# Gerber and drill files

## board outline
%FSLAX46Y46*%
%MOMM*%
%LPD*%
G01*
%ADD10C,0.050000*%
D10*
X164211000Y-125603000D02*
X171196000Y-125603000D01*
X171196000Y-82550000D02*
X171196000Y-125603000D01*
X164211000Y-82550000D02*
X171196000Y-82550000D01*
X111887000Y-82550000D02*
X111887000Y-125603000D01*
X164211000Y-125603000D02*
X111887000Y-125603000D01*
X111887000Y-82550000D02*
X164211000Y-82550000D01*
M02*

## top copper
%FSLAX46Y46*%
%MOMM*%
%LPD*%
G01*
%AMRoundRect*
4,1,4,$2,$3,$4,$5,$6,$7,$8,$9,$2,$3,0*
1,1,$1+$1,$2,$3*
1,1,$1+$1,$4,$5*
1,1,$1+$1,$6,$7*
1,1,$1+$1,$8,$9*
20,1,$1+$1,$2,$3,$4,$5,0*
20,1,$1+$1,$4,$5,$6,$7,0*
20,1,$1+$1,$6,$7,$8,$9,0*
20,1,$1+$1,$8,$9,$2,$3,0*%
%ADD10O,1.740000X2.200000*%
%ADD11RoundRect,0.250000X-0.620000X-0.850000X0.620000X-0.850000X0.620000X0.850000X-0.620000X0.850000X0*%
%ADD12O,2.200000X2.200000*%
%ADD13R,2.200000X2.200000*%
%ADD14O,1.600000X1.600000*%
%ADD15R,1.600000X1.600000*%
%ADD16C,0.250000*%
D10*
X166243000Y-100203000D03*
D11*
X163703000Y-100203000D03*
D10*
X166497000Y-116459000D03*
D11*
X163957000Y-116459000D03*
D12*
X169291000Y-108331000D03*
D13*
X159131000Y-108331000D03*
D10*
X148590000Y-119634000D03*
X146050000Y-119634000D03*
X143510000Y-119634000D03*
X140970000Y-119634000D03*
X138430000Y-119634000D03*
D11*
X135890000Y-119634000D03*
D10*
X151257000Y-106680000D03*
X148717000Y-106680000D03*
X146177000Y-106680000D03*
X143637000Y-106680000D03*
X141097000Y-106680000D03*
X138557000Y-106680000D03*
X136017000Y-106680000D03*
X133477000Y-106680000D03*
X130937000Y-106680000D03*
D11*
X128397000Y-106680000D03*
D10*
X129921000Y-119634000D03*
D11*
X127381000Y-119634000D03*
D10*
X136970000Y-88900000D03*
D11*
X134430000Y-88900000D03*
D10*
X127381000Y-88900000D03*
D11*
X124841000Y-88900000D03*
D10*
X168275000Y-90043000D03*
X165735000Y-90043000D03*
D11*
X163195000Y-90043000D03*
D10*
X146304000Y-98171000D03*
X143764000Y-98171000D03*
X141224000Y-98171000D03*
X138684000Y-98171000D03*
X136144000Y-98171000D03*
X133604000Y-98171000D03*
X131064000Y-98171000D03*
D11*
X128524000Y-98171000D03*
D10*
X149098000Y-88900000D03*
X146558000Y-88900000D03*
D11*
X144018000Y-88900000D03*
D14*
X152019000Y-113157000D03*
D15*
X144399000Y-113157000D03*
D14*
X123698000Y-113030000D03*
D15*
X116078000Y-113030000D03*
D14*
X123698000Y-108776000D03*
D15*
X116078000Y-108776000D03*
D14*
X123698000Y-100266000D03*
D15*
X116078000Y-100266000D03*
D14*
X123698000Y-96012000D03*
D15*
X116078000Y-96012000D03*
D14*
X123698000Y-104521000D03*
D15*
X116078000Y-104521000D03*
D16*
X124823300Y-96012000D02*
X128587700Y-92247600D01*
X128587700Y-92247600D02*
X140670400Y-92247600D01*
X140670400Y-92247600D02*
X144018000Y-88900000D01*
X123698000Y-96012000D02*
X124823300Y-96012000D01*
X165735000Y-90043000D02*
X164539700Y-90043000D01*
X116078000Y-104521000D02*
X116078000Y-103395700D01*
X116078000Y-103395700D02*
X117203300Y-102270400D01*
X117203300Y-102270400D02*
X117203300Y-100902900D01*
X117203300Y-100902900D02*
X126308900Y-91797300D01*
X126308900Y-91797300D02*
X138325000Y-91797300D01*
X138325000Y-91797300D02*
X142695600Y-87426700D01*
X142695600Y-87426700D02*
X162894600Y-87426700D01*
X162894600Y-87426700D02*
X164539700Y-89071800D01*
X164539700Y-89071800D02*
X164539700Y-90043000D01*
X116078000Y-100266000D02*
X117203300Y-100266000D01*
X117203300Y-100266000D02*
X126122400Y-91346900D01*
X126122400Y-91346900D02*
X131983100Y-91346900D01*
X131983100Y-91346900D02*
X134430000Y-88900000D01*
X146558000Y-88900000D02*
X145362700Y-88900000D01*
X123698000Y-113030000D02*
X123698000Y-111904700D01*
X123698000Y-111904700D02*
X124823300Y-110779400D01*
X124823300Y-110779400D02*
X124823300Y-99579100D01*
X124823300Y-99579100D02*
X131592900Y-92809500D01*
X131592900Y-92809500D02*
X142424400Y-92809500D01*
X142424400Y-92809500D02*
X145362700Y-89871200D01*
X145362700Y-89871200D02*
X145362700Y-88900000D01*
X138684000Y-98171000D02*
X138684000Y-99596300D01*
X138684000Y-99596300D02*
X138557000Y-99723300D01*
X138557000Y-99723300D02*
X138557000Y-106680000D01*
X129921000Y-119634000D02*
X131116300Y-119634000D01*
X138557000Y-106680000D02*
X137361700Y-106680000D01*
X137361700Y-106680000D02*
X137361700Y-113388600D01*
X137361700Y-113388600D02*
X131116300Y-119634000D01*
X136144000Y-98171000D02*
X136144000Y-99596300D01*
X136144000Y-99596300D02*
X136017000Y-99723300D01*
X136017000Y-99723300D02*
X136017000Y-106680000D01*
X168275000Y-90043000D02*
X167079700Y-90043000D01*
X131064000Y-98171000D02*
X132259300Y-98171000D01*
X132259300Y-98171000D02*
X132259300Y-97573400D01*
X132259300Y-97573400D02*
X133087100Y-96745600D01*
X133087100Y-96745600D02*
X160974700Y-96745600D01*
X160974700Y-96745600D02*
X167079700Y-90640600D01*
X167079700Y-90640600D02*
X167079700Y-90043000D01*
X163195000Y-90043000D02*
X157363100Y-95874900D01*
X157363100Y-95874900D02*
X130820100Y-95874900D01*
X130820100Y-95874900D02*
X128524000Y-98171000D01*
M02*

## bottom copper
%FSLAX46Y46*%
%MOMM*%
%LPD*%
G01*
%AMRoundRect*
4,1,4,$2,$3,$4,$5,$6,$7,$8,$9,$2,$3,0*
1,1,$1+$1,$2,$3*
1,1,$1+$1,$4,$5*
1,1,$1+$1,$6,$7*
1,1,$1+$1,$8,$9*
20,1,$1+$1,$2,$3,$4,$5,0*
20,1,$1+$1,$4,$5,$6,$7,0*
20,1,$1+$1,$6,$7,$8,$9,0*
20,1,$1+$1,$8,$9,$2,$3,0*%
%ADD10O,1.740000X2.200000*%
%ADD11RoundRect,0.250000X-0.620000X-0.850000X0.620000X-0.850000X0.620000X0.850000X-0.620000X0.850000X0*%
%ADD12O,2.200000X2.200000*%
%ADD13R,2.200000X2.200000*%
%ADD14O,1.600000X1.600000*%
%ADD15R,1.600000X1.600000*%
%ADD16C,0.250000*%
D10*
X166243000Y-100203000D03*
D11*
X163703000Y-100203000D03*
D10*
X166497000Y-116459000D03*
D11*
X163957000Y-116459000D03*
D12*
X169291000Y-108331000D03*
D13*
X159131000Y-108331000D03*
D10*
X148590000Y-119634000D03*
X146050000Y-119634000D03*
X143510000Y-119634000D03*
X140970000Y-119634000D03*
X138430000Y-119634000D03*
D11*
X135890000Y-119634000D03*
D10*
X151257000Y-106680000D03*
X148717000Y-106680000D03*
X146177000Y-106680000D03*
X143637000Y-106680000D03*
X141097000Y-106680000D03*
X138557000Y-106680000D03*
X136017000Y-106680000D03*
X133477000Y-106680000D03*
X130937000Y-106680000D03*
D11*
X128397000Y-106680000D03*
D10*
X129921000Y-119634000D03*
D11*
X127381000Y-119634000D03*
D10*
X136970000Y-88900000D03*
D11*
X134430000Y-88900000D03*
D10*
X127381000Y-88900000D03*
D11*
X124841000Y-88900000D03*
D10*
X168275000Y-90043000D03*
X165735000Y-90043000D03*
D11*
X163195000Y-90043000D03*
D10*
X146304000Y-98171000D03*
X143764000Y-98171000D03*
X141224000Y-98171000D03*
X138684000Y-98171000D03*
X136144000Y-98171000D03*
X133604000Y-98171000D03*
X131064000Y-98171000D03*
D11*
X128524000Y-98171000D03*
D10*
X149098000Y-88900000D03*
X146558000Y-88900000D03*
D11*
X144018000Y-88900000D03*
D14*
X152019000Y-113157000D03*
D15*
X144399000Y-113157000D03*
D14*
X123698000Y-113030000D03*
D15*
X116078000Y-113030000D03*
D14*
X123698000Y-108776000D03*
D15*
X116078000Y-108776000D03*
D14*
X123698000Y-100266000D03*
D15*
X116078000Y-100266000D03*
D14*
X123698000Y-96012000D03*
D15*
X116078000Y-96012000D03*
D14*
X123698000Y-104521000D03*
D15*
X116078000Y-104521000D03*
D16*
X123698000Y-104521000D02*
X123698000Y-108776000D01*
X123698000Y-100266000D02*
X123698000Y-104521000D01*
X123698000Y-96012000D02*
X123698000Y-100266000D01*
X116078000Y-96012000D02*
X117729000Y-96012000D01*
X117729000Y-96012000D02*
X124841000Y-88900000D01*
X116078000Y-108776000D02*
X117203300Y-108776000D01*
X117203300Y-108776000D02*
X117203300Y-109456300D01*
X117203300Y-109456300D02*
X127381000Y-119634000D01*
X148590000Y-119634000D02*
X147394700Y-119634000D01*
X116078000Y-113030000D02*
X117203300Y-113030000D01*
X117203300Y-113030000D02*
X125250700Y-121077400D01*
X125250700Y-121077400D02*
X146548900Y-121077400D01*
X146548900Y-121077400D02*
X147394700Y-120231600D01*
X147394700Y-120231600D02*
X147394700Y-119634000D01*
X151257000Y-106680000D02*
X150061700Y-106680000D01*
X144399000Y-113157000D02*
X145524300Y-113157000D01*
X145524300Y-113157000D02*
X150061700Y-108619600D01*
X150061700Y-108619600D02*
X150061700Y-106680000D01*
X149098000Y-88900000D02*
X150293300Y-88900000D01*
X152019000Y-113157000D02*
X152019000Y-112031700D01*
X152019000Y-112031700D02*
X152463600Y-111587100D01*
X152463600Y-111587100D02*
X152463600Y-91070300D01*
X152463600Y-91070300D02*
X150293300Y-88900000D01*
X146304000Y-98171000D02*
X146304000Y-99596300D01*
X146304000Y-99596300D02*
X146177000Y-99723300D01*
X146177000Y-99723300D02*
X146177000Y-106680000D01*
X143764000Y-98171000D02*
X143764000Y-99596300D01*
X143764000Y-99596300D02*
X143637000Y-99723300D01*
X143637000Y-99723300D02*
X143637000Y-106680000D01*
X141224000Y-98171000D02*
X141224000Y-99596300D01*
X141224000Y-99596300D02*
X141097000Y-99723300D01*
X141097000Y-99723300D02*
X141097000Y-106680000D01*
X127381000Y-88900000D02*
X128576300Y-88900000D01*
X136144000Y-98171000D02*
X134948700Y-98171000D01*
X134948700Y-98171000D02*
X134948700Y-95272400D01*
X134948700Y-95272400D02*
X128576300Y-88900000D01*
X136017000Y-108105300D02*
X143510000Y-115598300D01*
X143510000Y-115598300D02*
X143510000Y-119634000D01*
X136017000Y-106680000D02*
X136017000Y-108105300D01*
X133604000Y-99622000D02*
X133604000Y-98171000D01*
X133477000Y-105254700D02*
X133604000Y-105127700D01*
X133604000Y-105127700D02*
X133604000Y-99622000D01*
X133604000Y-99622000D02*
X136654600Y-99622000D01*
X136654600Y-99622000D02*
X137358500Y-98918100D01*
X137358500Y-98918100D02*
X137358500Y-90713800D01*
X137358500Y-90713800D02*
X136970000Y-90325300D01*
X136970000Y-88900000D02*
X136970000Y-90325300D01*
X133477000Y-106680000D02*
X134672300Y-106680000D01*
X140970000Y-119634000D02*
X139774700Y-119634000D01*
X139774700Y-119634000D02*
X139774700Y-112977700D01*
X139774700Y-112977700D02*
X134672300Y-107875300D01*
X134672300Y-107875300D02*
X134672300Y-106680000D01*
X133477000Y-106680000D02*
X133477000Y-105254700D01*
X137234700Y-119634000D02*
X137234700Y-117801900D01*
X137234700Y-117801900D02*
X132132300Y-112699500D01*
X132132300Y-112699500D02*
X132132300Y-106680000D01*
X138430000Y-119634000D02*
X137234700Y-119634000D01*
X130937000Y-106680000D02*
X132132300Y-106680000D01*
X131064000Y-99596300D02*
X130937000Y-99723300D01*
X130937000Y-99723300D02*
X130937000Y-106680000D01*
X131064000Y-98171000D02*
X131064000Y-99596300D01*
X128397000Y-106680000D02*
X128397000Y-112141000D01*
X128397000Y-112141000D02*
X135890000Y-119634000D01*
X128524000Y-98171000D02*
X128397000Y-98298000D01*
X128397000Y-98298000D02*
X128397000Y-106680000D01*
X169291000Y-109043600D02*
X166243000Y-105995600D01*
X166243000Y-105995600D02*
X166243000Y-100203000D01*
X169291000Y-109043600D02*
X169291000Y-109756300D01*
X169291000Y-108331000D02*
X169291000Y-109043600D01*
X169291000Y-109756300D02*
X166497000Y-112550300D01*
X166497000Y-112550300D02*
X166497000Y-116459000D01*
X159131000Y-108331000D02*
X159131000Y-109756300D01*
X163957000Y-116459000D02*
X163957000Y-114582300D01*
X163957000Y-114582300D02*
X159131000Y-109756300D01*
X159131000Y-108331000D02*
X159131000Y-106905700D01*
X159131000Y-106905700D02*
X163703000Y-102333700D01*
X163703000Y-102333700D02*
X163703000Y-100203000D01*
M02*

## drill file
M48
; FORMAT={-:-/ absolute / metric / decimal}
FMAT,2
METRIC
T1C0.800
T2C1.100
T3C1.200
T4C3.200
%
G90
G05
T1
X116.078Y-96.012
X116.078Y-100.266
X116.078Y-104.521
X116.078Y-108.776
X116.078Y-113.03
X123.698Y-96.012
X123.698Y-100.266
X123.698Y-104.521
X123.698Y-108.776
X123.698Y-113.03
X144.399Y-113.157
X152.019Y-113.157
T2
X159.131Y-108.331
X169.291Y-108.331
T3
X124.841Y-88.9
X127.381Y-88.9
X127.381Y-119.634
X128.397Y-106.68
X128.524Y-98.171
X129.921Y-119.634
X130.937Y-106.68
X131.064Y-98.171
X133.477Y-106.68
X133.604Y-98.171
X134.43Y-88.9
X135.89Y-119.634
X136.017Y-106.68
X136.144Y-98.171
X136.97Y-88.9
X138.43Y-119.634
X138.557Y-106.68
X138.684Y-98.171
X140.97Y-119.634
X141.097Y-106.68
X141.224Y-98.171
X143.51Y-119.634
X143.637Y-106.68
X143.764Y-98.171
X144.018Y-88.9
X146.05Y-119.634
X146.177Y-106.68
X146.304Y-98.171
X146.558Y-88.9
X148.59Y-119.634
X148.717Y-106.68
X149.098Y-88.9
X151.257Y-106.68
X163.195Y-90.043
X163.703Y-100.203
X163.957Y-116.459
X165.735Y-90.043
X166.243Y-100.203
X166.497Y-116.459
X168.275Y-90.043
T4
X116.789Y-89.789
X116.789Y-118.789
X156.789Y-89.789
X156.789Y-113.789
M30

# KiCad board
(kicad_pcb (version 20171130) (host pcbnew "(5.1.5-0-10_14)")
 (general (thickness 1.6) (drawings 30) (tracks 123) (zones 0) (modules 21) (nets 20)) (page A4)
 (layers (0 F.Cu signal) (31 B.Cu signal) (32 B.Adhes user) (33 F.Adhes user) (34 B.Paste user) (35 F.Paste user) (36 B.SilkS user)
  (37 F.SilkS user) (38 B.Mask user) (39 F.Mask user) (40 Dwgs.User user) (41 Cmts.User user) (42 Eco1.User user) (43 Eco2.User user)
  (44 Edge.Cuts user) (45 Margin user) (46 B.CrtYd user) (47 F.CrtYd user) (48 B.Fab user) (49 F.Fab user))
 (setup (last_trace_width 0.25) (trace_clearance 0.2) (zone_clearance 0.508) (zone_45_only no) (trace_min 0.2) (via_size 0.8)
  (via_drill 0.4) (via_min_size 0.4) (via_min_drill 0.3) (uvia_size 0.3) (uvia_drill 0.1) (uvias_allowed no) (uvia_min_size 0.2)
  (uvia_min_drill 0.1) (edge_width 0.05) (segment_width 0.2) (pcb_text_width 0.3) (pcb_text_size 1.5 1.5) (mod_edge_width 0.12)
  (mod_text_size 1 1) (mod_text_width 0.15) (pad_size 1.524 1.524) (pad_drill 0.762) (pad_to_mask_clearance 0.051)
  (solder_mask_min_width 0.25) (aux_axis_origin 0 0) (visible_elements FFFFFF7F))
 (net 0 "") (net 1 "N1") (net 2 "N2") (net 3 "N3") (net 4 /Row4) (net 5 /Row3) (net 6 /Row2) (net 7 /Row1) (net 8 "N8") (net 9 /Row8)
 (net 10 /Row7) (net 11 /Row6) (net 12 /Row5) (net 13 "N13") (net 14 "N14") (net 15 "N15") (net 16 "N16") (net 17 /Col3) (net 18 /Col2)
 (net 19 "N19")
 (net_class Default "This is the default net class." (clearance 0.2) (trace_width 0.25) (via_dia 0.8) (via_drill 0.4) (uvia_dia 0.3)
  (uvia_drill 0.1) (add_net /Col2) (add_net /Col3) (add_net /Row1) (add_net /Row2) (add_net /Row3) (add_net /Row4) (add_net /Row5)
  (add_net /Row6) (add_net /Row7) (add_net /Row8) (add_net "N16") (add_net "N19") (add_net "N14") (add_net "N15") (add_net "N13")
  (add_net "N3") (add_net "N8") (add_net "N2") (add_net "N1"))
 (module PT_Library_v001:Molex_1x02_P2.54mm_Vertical (layer F.Cu) (at 163.703 100.203)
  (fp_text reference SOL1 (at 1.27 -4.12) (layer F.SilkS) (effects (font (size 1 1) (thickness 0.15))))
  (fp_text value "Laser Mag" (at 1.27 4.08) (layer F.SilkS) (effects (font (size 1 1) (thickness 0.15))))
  (pad 2 thru_hole oval (at 2.54 0) (size 1.74 2.2) (drill 1.2) (layers *.Cu *.Mask) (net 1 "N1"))
  (pad 1 thru_hole roundrect (at 0 0) (size 1.74 2.2) (drill 1.2) (layers *.Cu *.Mask) (roundrect_rratio 0.143678) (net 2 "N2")))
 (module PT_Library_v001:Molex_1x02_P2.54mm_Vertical (layer F.Cu) (at 163.957 116.459)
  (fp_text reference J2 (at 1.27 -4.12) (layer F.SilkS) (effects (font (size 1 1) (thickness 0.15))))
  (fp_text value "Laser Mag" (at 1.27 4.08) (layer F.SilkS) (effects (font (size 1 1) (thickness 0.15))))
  (pad 2 thru_hole oval (at 2.54 0) (size 1.74 2.2) (drill 1.2) (layers *.Cu *.Mask) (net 1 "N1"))
  (pad 1 thru_hole roundrect (at 0 0) (size 1.74 2.2) (drill 1.2) (layers *.Cu *.Mask) (roundrect_rratio 0.143678) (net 2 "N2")))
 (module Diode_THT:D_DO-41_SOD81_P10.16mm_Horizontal (layer F.Cu) (at 159.131 108.331)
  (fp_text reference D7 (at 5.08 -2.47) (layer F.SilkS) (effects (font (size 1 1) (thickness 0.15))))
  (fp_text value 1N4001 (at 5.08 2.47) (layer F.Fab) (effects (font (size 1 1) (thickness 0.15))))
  (pad 2 thru_hole oval (at 10.16 0) (size 2.2 2.2) (drill 1.1) (layers *.Cu *.Mask) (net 1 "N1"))
  (pad 1 thru_hole rect (at 0 0) (size 2.2 2.2) (drill 1.1) (layers *.Cu *.Mask) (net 2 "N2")))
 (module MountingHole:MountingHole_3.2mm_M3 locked (layer F.Cu) (at 116.789 89.789)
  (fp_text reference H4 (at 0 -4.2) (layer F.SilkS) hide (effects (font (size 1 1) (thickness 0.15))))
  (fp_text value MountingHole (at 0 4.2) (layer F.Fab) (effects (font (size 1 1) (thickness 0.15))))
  (pad 1 np_thru_hole circle (at 0 0) (size 3.2 3.2) (drill 3.2) (layers *.Cu *.Mask)))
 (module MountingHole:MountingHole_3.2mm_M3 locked (layer F.Cu) (at 156.789 89.789)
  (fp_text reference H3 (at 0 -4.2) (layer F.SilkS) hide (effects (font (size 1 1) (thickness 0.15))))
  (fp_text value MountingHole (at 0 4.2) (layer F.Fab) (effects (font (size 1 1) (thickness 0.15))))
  (pad 1 np_thru_hole circle (at 0 0) (size 3.2 3.2) (drill 3.2) (layers *.Cu *.Mask)))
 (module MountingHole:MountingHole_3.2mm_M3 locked (layer F.Cu) (at 156.789 113.789)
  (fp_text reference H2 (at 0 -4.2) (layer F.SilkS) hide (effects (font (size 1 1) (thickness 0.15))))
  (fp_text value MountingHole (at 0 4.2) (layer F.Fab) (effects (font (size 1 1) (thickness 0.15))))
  (pad 1 np_thru_hole circle (at 0 0) (size 3.2 3.2) (drill 3.2) (layers *.Cu *.Mask)))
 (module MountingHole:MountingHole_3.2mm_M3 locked (layer F.Cu) (at 116.789 118.789)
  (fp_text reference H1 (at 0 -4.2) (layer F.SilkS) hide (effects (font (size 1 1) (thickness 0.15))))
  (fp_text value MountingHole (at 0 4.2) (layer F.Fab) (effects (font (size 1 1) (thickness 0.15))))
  (pad 1 np_thru_hole circle (at 0 0) (size 3.2 3.2) (drill 3.2) (layers *.Cu *.Mask)))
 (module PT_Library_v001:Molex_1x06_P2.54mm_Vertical (layer F.Cu) (at 135.89 119.634)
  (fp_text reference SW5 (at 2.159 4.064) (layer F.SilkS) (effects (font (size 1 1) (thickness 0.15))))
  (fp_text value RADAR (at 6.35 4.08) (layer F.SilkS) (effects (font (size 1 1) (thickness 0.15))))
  (pad 6 thru_hole oval (at 12.7 0) (size 1.74 2.2) (drill 1.2) (layers *.Cu *.Mask) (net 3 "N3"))
  (pad 5 thru_hole oval (at 10.16 0) (size 1.74 2.2) (drill 1.2) (layers *.Cu *.Mask))
  (pad 4 thru_hole oval (at 7.62 0) (size 1.74 2.2) (drill 1.2) (layers *.Cu *.Mask) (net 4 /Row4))
  (pad 3 thru_hole oval (at 5.08 0) (size 1.74 2.2) (drill 1.2) (layers *.Cu *.Mask) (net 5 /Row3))
  (pad 2 thru_hole oval (at 2.54 0) (size 1.74 2.2) (drill 1.2) (layers *.Cu *.Mask) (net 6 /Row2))
  (pad 1 thru_hole roundrect (at 0 0) (size 1.74 2.2) (drill 1.2) (layers *.Cu *.Mask) (roundrect_rratio 0.143678) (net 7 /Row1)))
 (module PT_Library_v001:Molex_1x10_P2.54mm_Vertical (layer F.Cu) (at 128.397 106.68)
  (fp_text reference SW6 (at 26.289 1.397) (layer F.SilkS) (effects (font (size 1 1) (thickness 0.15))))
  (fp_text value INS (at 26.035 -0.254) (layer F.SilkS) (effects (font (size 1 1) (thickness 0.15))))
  (pad 10 thru_hole oval (at 22.86 0) (size 1.74 2.2) (drill 1.2) (layers *.Cu *.Mask) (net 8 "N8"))
  (pad 9 thru_hole oval (at 20.32 0) (size 1.74 2.2) (drill 1.2) (layers *.Cu *.Mask))
  (pad 8 thru_hole oval (at 17.78 0) (size 1.74 2.2) (drill 1.2) (layers *.Cu *.Mask) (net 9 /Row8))
  (pad 7 thru_hole oval (at 15.24 0) (size 1.74 2.2) (drill 1.2) (layers *.Cu *.Mask) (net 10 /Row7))
  (pad 6 thru_hole oval (at 12.7 0) (size 1.74 2.2) (drill 1.2) (layers *.Cu *.Mask) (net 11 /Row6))
  (pad 5 thru_hole oval (at 10.16 0) (size 1.74 2.2) (drill 1.2) (layers *.Cu *.Mask) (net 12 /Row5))
  (pad 4 thru_hole oval (at 7.62 0) (size 1.74 2.2) (drill 1.2) (layers *.Cu *.Mask) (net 4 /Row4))
  (pad 3 thru_hole oval (at 5.08 0) (size 1.74 2.2) (drill 1.2) (layers *.Cu *.Mask) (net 5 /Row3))
  (pad 2 thru_hole oval (at 2.54 0) (size 1.74 2.2) (drill 1.2) (layers *.Cu *.Mask) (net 6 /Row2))
  (pad 1 thru_hole roundrect (at 0 0) (size 1.74 2.2) (drill 1.2) (layers *.Cu *.Mask) (roundrect_rratio 0.143678) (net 7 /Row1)))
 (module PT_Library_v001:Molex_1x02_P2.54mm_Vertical (layer F.Cu) (at 127.381 119.634)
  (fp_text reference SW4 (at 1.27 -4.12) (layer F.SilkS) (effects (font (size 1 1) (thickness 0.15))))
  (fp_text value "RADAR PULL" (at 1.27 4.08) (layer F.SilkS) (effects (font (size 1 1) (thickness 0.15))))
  (pad 2 thru_hole oval (at 2.54 0) (size 1.74 2.2) (drill 1.2) (layers *.Cu *.Mask) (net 12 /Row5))
  (pad 1 thru_hole roundrect (at 0 0) (size 1.74 2.2) (drill 1.2) (layers *.Cu *.Mask) (roundrect_rratio 0.143678) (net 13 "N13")))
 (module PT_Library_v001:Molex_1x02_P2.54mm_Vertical (layer F.Cu) (at 134.43 88.9)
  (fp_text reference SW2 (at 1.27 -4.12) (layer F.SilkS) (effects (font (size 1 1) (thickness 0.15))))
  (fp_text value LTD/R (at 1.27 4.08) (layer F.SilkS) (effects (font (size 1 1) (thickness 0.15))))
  (pad 2 thru_hole oval (at 2.54 0) (size 1.74 2.2) (drill 1.2) (layers *.Cu *.Mask) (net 5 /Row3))
  (pad 1 thru_hole roundrect (at 0 0) (size 1.74 2.2) (drill 1.2) (layers *.Cu *.Mask) (roundrect_rratio 0.143678) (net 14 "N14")))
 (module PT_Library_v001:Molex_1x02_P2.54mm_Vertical (layer F.Cu) (at 124.841 88.9)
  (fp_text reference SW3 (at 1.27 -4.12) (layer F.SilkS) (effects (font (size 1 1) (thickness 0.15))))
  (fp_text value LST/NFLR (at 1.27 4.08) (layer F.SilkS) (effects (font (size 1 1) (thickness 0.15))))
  (pad 2 thru_hole oval (at 2.54 0) (size 1.74 2.2) (drill 1.2) (layers *.Cu *.Mask) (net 4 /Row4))
  (pad 1 thru_hole roundrect (at 0 0) (size 1.74 2.2) (drill 1.2) (layers *.Cu *.Mask) (roundrect_rratio 0.143678) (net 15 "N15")))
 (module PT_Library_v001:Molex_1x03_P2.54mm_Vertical (layer F.Cu) (at 163.195 90.043)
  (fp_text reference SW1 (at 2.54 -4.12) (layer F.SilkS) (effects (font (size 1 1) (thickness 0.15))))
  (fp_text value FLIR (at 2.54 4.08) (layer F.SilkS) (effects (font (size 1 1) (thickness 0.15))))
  (pad 3 thru_hole oval (at 5.08 0) (size 1.74 2.2) (drill 1.2) (layers *.Cu *.Mask) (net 6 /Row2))
  (pad 2 thru_hole oval (at 2.54 0) (size 1.74 2.2) (drill 1.2) (layers *.Cu *.Mask) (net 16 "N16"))
  (pad 1 thru_hole roundrect (at 0 0) (size 1.74 2.2) (drill 1.2) (layers *.Cu *.Mask) (roundrect_rratio 0.143678) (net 7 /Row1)))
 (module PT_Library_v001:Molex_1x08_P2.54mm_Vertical (layer F.Cu) (at 128.524 98.171)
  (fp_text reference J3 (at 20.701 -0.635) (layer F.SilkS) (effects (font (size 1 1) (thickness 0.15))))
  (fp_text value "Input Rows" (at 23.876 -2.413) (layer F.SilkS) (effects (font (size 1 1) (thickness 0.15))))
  (pad 8 thru_hole oval (at 17.78 0) (size 1.74 2.2) (drill 1.2) (layers *.Cu *.Mask) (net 9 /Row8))
  (pad 7 thru_hole oval (at 15.24 0) (size 1.74 2.2) (drill 1.2) (layers *.Cu *.Mask) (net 10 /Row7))
  (pad 6 thru_hole oval (at 12.7 0) (size 1.74 2.2) (drill 1.2) (layers *.Cu *.Mask) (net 11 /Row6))
  (pad 5 thru_hole oval (at 10.16 0) (size 1.74 2.2) (drill 1.2) (layers *.Cu *.Mask) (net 12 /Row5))
  (pad 4 thru_hole oval (at 7.62 0) (size 1.74 2.2) (drill 1.2) (layers *.Cu *.Mask) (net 4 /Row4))
  (pad 3 thru_hole oval (at 5.08 0) (size 1.74 2.2) (drill 1.2) (layers *.Cu *.Mask) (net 5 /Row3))
  (pad 2 thru_hole oval (at 2.54 0) (size 1.74 2.2) (drill 1.2) (layers *.Cu *.Mask) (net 6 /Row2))
  (pad 1 thru_hole roundrect (at 0 0) (size 1.74 2.2) (drill 1.2) (layers *.Cu *.Mask) (roundrect_rratio 0.143678) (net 7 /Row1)))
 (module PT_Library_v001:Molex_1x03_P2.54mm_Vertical (layer F.Cu) (at 144.018 88.9)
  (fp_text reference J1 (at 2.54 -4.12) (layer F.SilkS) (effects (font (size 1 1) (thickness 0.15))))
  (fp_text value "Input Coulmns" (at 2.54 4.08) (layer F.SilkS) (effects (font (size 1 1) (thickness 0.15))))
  (pad 3 thru_hole oval (at 5.08 0) (size 1.74 2.2) (drill 1.2) (layers *.Cu *.Mask) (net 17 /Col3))
  (pad 2 thru_hole oval (at 2.54 0) (size 1.74 2.2) (drill 1.2) (layers *.Cu *.Mask) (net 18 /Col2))
  (pad 1 thru_hole roundrect (at 0 0) (size 1.74 2.2) (drill 1.2) (layers *.Cu *.Mask) (roundrect_rratio 0.143678) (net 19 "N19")))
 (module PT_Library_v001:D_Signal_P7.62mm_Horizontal (layer F.Cu) (at 144.399 113.157)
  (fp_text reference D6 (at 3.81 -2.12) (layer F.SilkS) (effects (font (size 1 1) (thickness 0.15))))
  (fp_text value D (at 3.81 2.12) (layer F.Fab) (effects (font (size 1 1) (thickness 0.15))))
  (pad 2 thru_hole oval (at 7.62 0) (size 1.6 1.6) (drill 0.8) (layers *.Cu *.Mask) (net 17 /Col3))
  (pad 1 thru_hole rect (at 0 0) (size 1.6 1.6) (drill 0.8) (layers *.Cu *.Mask) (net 8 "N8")))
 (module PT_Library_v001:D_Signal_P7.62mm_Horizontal (layer F.Cu) (at 116.078 113.03)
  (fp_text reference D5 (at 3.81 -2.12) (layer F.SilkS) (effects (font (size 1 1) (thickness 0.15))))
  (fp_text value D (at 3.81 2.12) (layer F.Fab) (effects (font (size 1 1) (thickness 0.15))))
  (pad 2 thru_hole oval (at 7.62 0) (size 1.6 1.6) (drill 0.8) (layers *.Cu *.Mask) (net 18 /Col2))
  (pad 1 thru_hole rect (at 0 0) (size 1.6 1.6) (drill 0.8) (layers *.Cu *.Mask) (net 3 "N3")))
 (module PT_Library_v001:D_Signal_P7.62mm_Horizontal (layer F.Cu) (at 116.078 108.776)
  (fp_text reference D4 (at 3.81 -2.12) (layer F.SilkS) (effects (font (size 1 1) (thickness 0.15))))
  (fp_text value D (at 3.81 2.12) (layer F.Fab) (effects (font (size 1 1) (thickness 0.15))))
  (pad 2 thru_hole oval (at 7.62 0) (size 1.6 1.6) (drill 0.8) (layers *.Cu *.Mask) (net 19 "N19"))
  (pad 1 thru_hole rect (at 0 0) (size 1.6 1.6) (drill 0.8) (layers *.Cu *.Mask) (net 13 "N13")))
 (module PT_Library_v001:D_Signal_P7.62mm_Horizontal (layer F.Cu) (at 116.078 100.266)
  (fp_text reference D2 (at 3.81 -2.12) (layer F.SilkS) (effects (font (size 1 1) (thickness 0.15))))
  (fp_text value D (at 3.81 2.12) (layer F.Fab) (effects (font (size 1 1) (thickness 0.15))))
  (pad 2 thru_hole oval (at 7.62 0) (size 1.6 1.6) (drill 0.8) (layers *.Cu *.Mask) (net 19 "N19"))
  (pad 1 thru_hole rect (at 0 0) (size 1.6 1.6) (drill 0.8) (layers *.Cu *.Mask) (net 14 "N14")))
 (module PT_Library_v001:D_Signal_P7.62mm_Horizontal (layer F.Cu) (at 116.078 96.012)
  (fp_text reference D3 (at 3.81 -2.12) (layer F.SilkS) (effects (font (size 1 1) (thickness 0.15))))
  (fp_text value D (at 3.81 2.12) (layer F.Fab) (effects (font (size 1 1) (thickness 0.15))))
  (pad 2 thru_hole oval (at 7.62 0) (size 1.6 1.6) (drill 0.8) (layers *.Cu *.Mask) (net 19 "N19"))
  (pad 1 thru_hole rect (at 0 0) (size 1.6 1.6) (drill 0.8) (layers *.Cu *.Mask) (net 15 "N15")))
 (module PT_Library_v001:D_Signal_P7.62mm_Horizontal (layer F.Cu) (at 116.078 104.521)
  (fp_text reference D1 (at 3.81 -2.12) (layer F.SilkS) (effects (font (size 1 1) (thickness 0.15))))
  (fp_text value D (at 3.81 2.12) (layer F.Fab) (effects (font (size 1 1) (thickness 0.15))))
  (pad 2 thru_hole oval (at 7.62 0) (size 1.6 1.6) (drill 0.8) (layers *.Cu *.Mask) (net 19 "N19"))
  (pad 1 thru_hole rect (at 0 0) (size 1.6 1.6) (drill 0.8) (layers *.Cu *.Mask) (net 16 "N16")))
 (gr_line (start 164.211 125.603) (end 171.196 125.603) (layer Edge.Cuts) (width 0.05))
 (gr_line (start 171.196 82.55) (end 171.196 125.603) (layer Edge.Cuts) (width 0.05))
 (gr_line (start 164.211 82.55) (end 171.196 82.55) (layer Edge.Cuts) (width 0.05))
 (gr_line (start 111.887 82.55) (end 111.887 125.603) (layer Edge.Cuts) (width 0.05))
 (gr_line (start 164.211 125.603) (end 111.887 125.603) (layer Edge.Cuts) (width 0.05))
 (gr_line (start 111.887 82.55) (end 164.211 82.55) (layer Edge.Cuts) (width 0.05))
 (segment (start 124.8233 96.012) (end 128.5877 92.2476) (width 0.25) (layer F.Cu) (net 19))
 (segment (start 128.5877 92.2476) (end 140.6704 92.2476) (width 0.25) (layer F.Cu) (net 19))
 (segment (start 140.6704 92.2476) (end 144.018 88.9) (width 0.25) (layer F.Cu) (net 19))
 (segment (start 123.698 96.012) (end 124.8233 96.012) (width 0.25) (layer F.Cu) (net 19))
 (segment (start 123.698 104.521) (end 123.698 108.776) (width 0.25) (layer B.Cu) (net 19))
 (segment (start 123.698 100.266) (end 123.698 104.521) (width 0.25) (layer B.Cu) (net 19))
 (segment (start 123.698 96.012) (end 123.698 100.266) (width 0.25) (layer B.Cu) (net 19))
 (segment (start 165.735 90.043) (end 164.5397 90.043) (width 0.25) (layer F.Cu) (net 16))
 (segment (start 116.078 104.521) (end 116.078 103.3957) (width 0.25) (layer F.Cu) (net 16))
 (segment (start 116.078 103.3957) (end 117.2033 102.2704) (width 0.25) (layer F.Cu) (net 16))
 (segment (start 117.2033 102.2704) (end 117.2033 100.9029) (width 0.25) (layer F.Cu) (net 16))
 (segment (start 117.2033 100.9029) (end 126.3089 91.7973) (width 0.25) (layer F.Cu) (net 16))
 (segment (start 126.3089 91.7973) (end 138.325 91.7973) (width 0.25) (layer F.Cu) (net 16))
 (segment (start 138.325 91.7973) (end 142.6956 87.4267) (width 0.25) (layer F.Cu) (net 16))
 (segment (start 142.6956 87.4267) (end 162.8946 87.4267) (width 0.25) (layer F.Cu) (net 16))
 (segment (start 162.8946 87.4267) (end 164.5397 89.0718) (width 0.25) (layer F.Cu) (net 16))
 (segment (start 164.5397 89.0718) (end 164.5397 90.043) (width 0.25) (layer F.Cu) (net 16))
 (segment (start 116.078 100.266) (end 117.2033 100.266) (width 0.25) (layer F.Cu) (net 14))
 (segment (start 117.2033 100.266) (end 126.1224 91.3469) (width 0.25) (layer F.Cu) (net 14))
 (segment (start 126.1224 91.3469) (end 131.9831 91.3469) (width 0.25) (layer F.Cu) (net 14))
 (segment (start 131.9831 91.3469) (end 134.43 88.9) (width 0.25) (layer F.Cu) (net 14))
 (segment (start 116.078 96.012) (end 117.729 96.012) (width 0.25) (layer B.Cu) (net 15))
 (segment (start 117.729 96.012) (end 124.841 88.9) (width 0.25) (layer B.Cu) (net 15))
 (segment (start 116.078 108.776) (end 117.2033 108.776) (width 0.25) (layer B.Cu) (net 13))
 (segment (start 117.2033 108.776) (end 117.2033 109.4563) (width 0.25) (layer B.Cu) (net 13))
 (segment (start 117.2033 109.4563) (end 127.381 119.634) (width 0.25) (layer B.Cu) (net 13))
 (segment (start 148.59 119.634) (end 147.3947 119.634) (width 0.25) (layer B.Cu) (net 3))
 (segment (start 116.078 113.03) (end 117.2033 113.03) (width 0.25) (layer B.Cu) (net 3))
 (segment (start 117.2033 113.03) (end 125.2507 121.0774) (width 0.25) (layer B.Cu) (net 3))
 (segment (start 125.2507 121.0774) (end 146.5489 121.0774) (width 0.25) (layer B.Cu) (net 3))
 (segment (start 146.5489 121.0774) (end 147.3947 120.2316) (width 0.25) (layer B.Cu) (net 3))
 (segment (start 147.3947 120.2316) (end 147.3947 119.634) (width 0.25) (layer B.Cu) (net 3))
 (segment (start 146.558 88.9) (end 145.3627 88.9) (width 0.25) (layer F.Cu) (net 18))
 (segment (start 123.698 113.03) (end 123.698 111.9047) (width 0.25) (layer F.Cu) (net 18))
 (segment (start 123.698 111.9047) (end 124.8233 110.7794) (width 0.25) (layer F.Cu) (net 18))
 (segment (start 124.8233 110.7794) (end 124.8233 99.5791) (width 0.25) (layer F.Cu) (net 18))
 (segment (start 124.8233 99.5791) (end 131.5929 92.8095) (width 0.25) (layer F.Cu) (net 18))
 (segment (start 131.5929 92.8095) (end 142.4244 92.8095) (width 0.25) (layer F.Cu) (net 18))
 (segment (start 142.4244 92.8095) (end 145.3627 89.8712) (width 0.25) (layer F.Cu) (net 18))
 (segment (start 145.3627 89.8712) (end 145.3627 88.9) (width 0.25) (layer F.Cu) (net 18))
 (segment (start 151.257 106.68) (end 150.0617 106.68) (width 0.25) (layer B.Cu) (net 8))
 (segment (start 144.399 113.157) (end 145.5243 113.157) (width 0.25) (layer B.Cu) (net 8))
 (segment (start 145.5243 113.157) (end 150.0617 108.6196) (width 0.25) (layer B.Cu) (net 8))
 (segment (start 150.0617 108.6196) (end 150.0617 106.68) (width 0.25) (layer B.Cu) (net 8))
 (segment (start 149.098 88.9) (end 150.2933 88.9) (width 0.25) (layer B.Cu) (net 17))
 (segment (start 152.019 113.157) (end 152.019 112.0317) (width 0.25) (layer B.Cu) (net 17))
 (segment (start 152.019 112.0317) (end 152.4636 111.5871) (width 0.25) (layer B.Cu) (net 17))
 (segment (start 152.4636 111.5871) (end 152.4636 91.0703) (width 0.25) (layer B.Cu) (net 17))
 (segment (start 152.4636 91.0703) (end 150.2933 88.9) (width 0.25) (layer B.Cu) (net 17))
 (segment (start 146.304 98.171) (end 146.304 99.5963) (width 0.25) (layer B.Cu) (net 9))
 (segment (start 146.304 99.5963) (end 146.177 99.7233) (width 0.25) (layer B.Cu) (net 9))
 (segment (start 146.177 99.7233) (end 146.177 106.68) (width 0.25) (layer B.Cu) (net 9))
 (segment (start 143.764 98.171) (end 143.764 99.5963) (width 0.25) (layer B.Cu) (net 10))
 (segment (start 143.764 99.5963) (end 143.637 99.7233) (width 0.25) (layer B.Cu) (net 10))
 (segment (start 143.637 99.7233) (end 143.637 106.68) (width 0.25) (layer B.Cu) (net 10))
 (segment (start 141.224 98.171) (end 141.224 99.5963) (width 0.25) (layer B.Cu) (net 11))
 (segment (start 141.224 99.5963) (end 141.097 99.7233) (width 0.25) (layer B.Cu) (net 11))
 (segment (start 141.097 99.7233) (end 141.097 106.68) (width 0.25) (layer B.Cu) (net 11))
 (segment (start 138.684 98.171) (end 138.684 99.5963) (width 0.25) (layer F.Cu) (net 12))
 (segment (start 138.684 99.5963) (end 138.557 99.7233) (width 0.25) (layer F.Cu) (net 12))
 (segment (start 138.557 99.7233) (end 138.557 106.68) (width 0.25) (layer F.Cu) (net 12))
 (segment (start 129.921 119.634) (end 131.1163 119.634) (width 0.25) (layer F.Cu) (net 12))
 (segment (start 138.557 106.68) (end 137.3617 106.68) (width 0.25) (layer F.Cu) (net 12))
 (segment (start 137.3617 106.68) (end 137.3617 113.3886) (width 0.25) (layer F.Cu) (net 12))
 (segment (start 137.3617 113.3886) (end 131.1163 119.634) (width 0.25) (layer F.Cu) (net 12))
 (segment (start 127.381 88.9) (end 128.5763 88.9) (width 0.25) (layer B.Cu) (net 4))
 (segment (start 136.144 98.171) (end 134.9487 98.171) (width 0.25) (layer B.Cu) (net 4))
 (segment (start 134.9487 98.171) (end 134.9487 95.2724) (width 0.25) (layer B.Cu) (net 4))
 (segment (start 134.9487 95.2724) (end 128.5763 88.9) (width 0.25) (layer B.Cu) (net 4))
 (segment (start 136.144 98.171) (end 136.144 99.5963) (width 0.25) (layer F.Cu) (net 4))
 (segment (start 136.144 99.5963) (end 136.017 99.7233) (width 0.25) (layer F.Cu) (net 4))
 (segment (start 136.017 99.7233) (end 136.017 106.68) (width 0.25) (layer F.Cu) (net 4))
 (segment (start 136.017 108.1053) (end 143.51 115.5983) (width 0.25) (layer B.Cu) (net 4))
 (segment (start 143.51 115.5983) (end 143.51 119.634) (width 0.25) (layer B.Cu) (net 4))
 (segment (start 136.017 106.68) (end 136.017 108.1053) (width 0.25) (layer B.Cu) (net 4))
 (segment (start 133.604 99.622) (end 133.604 98.171) (width 0.25) (layer B.Cu) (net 5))
 (segment (start 133.477 105.2547) (end 133.604 105.1277) (width 0.25) (layer B.Cu) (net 5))
 (segment (start 133.604 105.1277) (end 133.604 99.622) (width 0.25) (layer B.Cu) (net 5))
 (segment (start 133.604 99.622) (end 136.6546 99.622) (width 0.25) (layer B.Cu) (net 5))
 (segment (start 136.6546 99.622) (end 137.3585 98.9181) (width 0.25) (layer B.Cu) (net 5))
 (segment (start 137.3585 98.9181) (end 137.3585 90.7138) (width 0.25) (layer B.Cu) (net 5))
 (segment (start 137.3585 90.7138) (end 136.97 90.3253) (width 0.25) (layer B.Cu) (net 5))
 (segment (start 136.97 88.9) (end 136.97 90.3253) (width 0.25) (layer B.Cu) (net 5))
 (segment (start 133.477 106.68) (end 134.6723 106.68) (width 0.25) (layer B.Cu) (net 5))
 (segment (start 140.97 119.634) (end 139.7747 119.634) (width 0.25) (layer B.Cu) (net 5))
 (segment (start 139.7747 119.634) (end 139.7747 112.9777) (width 0.25) (layer B.Cu) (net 5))
 (segment (start 139.7747 112.9777) (end 134.6723 107.8753) (width 0.25) (layer B.Cu) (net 5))
 (segment (start 134.6723 107.8753) (end 134.6723 106.68) (width 0.25) (layer B.Cu) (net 5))
 (segment (start 133.477 106.68) (end 133.477 105.2547) (width 0.25) (layer B.Cu) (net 5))
 (segment (start 137.2347 119.634) (end 137.2347 117.8019) (width 0.25) (layer B.Cu) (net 6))
 (segment (start 137.2347 117.8019) (end 132.1323 112.6995) (width 0.25) (layer B.Cu) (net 6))
 (segment (start 132.1323 112.6995) (end 132.1323 106.68) (width 0.25) (layer B.Cu) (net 6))
 (segment (start 168.275 90.043) (end 167.0797 90.043) (width 0.25) (layer F.Cu) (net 6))
 (segment (start 131.064 98.171) (end 132.2593 98.171) (width 0.25) (layer F.Cu) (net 6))
 (segment (start 132.2593 98.171) (end 132.2593 97.5734) (width 0.25) (layer F.Cu) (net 6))
 (segment (start 132.2593 97.5734) (end 133.0871 96.7456) (width 0.25) (layer F.Cu) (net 6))
 (segment (start 133.0871 96.7456) (end 160.9747 96.7456) (width 0.25) (layer F.Cu) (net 6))
 (segment (start 160.9747 96.7456) (end 167.0797 90.6406) (width 0.25) (layer F.Cu) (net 6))
 (segment (start 167.0797 90.6406) (end 167.0797 90.043) (width 0.25) (layer F.Cu) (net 6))
 (segment (start 138.43 119.634) (end 137.2347 119.634) (width 0.25) (layer B.Cu) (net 6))
 (segment (start 130.937 106.68) (end 132.1323 106.68) (width 0.25) (layer B.Cu) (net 6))
 (segment (start 131.064 99.5963) (end 130.937 99.7233) (width 0.25) (layer B.Cu) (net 6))
 (segment (start 130.937 99.7233) (end 130.937 106.68) (width 0.25) (layer B.Cu) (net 6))
 (segment (start 131.064 98.171) (end 131.064 99.5963) (width 0.25) (layer B.Cu) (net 6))
 (segment (start 128.397 106.68) (end 128.397 112.141) (width 0.25) (layer B.Cu) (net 7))
 (segment (start 128.397 112.141) (end 135.89 119.634) (width 0.25) (layer B.Cu) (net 7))
 (segment (start 128.524 98.171) (end 128.397 98.298) (width 0.25) (layer B.Cu) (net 7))
 (segment (start 128.397 98.298) (end 128.397 106.68) (width 0.25) (layer B.Cu) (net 7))
 (segment (start 163.195 90.043) (end 157.3631 95.8749) (width 0.25) (layer F.Cu) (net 7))
 (segment (start 157.3631 95.8749) (end 130.8201 95.8749) (width 0.25) (layer F.Cu) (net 7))
 (segment (start 130.8201 95.8749) (end 128.524 98.171) (width 0.25) (layer F.Cu) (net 7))
 (segment (start 169.291 109.0436) (end 166.243 105.9956) (width 0.25) (layer B.Cu) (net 1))
 (segment (start 166.243 105.9956) (end 166.243 100.203) (width 0.25) (layer B.Cu) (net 1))
 (segment (start 169.291 109.0436) (end 169.291 109.7563) (width 0.25) (layer B.Cu) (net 1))
 (segment (start 169.291 108.331) (end 169.291 109.0436) (width 0.25) (layer B.Cu) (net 1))
 (segment (start 169.291 109.7563) (end 166.497 112.5503) (width 0.25) (layer B.Cu) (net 1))
 (segment (start 166.497 112.5503) (end 166.497 116.459) (width 0.25) (layer B.Cu) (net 1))
 (segment (start 159.131 108.331) (end 159.131 109.7563) (width 0.25) (layer B.Cu) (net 2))
 (segment (start 163.957 116.459) (end 163.957 114.5823) (width 0.25) (layer B.Cu) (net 2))
 (segment (start 163.957 114.5823) (end 159.131 109.7563) (width 0.25) (layer B.Cu) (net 2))
 (segment (start 159.131 108.331) (end 159.131 106.9057) (width 0.25) (layer B.Cu) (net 2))
 (segment (start 159.131 106.9057) (end 163.703 102.3337) (width 0.25) (layer B.Cu) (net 2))
 (segment (start 163.703 102.3337) (end 163.703 100.203) (width 0.25) (layer B.Cu) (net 2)))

